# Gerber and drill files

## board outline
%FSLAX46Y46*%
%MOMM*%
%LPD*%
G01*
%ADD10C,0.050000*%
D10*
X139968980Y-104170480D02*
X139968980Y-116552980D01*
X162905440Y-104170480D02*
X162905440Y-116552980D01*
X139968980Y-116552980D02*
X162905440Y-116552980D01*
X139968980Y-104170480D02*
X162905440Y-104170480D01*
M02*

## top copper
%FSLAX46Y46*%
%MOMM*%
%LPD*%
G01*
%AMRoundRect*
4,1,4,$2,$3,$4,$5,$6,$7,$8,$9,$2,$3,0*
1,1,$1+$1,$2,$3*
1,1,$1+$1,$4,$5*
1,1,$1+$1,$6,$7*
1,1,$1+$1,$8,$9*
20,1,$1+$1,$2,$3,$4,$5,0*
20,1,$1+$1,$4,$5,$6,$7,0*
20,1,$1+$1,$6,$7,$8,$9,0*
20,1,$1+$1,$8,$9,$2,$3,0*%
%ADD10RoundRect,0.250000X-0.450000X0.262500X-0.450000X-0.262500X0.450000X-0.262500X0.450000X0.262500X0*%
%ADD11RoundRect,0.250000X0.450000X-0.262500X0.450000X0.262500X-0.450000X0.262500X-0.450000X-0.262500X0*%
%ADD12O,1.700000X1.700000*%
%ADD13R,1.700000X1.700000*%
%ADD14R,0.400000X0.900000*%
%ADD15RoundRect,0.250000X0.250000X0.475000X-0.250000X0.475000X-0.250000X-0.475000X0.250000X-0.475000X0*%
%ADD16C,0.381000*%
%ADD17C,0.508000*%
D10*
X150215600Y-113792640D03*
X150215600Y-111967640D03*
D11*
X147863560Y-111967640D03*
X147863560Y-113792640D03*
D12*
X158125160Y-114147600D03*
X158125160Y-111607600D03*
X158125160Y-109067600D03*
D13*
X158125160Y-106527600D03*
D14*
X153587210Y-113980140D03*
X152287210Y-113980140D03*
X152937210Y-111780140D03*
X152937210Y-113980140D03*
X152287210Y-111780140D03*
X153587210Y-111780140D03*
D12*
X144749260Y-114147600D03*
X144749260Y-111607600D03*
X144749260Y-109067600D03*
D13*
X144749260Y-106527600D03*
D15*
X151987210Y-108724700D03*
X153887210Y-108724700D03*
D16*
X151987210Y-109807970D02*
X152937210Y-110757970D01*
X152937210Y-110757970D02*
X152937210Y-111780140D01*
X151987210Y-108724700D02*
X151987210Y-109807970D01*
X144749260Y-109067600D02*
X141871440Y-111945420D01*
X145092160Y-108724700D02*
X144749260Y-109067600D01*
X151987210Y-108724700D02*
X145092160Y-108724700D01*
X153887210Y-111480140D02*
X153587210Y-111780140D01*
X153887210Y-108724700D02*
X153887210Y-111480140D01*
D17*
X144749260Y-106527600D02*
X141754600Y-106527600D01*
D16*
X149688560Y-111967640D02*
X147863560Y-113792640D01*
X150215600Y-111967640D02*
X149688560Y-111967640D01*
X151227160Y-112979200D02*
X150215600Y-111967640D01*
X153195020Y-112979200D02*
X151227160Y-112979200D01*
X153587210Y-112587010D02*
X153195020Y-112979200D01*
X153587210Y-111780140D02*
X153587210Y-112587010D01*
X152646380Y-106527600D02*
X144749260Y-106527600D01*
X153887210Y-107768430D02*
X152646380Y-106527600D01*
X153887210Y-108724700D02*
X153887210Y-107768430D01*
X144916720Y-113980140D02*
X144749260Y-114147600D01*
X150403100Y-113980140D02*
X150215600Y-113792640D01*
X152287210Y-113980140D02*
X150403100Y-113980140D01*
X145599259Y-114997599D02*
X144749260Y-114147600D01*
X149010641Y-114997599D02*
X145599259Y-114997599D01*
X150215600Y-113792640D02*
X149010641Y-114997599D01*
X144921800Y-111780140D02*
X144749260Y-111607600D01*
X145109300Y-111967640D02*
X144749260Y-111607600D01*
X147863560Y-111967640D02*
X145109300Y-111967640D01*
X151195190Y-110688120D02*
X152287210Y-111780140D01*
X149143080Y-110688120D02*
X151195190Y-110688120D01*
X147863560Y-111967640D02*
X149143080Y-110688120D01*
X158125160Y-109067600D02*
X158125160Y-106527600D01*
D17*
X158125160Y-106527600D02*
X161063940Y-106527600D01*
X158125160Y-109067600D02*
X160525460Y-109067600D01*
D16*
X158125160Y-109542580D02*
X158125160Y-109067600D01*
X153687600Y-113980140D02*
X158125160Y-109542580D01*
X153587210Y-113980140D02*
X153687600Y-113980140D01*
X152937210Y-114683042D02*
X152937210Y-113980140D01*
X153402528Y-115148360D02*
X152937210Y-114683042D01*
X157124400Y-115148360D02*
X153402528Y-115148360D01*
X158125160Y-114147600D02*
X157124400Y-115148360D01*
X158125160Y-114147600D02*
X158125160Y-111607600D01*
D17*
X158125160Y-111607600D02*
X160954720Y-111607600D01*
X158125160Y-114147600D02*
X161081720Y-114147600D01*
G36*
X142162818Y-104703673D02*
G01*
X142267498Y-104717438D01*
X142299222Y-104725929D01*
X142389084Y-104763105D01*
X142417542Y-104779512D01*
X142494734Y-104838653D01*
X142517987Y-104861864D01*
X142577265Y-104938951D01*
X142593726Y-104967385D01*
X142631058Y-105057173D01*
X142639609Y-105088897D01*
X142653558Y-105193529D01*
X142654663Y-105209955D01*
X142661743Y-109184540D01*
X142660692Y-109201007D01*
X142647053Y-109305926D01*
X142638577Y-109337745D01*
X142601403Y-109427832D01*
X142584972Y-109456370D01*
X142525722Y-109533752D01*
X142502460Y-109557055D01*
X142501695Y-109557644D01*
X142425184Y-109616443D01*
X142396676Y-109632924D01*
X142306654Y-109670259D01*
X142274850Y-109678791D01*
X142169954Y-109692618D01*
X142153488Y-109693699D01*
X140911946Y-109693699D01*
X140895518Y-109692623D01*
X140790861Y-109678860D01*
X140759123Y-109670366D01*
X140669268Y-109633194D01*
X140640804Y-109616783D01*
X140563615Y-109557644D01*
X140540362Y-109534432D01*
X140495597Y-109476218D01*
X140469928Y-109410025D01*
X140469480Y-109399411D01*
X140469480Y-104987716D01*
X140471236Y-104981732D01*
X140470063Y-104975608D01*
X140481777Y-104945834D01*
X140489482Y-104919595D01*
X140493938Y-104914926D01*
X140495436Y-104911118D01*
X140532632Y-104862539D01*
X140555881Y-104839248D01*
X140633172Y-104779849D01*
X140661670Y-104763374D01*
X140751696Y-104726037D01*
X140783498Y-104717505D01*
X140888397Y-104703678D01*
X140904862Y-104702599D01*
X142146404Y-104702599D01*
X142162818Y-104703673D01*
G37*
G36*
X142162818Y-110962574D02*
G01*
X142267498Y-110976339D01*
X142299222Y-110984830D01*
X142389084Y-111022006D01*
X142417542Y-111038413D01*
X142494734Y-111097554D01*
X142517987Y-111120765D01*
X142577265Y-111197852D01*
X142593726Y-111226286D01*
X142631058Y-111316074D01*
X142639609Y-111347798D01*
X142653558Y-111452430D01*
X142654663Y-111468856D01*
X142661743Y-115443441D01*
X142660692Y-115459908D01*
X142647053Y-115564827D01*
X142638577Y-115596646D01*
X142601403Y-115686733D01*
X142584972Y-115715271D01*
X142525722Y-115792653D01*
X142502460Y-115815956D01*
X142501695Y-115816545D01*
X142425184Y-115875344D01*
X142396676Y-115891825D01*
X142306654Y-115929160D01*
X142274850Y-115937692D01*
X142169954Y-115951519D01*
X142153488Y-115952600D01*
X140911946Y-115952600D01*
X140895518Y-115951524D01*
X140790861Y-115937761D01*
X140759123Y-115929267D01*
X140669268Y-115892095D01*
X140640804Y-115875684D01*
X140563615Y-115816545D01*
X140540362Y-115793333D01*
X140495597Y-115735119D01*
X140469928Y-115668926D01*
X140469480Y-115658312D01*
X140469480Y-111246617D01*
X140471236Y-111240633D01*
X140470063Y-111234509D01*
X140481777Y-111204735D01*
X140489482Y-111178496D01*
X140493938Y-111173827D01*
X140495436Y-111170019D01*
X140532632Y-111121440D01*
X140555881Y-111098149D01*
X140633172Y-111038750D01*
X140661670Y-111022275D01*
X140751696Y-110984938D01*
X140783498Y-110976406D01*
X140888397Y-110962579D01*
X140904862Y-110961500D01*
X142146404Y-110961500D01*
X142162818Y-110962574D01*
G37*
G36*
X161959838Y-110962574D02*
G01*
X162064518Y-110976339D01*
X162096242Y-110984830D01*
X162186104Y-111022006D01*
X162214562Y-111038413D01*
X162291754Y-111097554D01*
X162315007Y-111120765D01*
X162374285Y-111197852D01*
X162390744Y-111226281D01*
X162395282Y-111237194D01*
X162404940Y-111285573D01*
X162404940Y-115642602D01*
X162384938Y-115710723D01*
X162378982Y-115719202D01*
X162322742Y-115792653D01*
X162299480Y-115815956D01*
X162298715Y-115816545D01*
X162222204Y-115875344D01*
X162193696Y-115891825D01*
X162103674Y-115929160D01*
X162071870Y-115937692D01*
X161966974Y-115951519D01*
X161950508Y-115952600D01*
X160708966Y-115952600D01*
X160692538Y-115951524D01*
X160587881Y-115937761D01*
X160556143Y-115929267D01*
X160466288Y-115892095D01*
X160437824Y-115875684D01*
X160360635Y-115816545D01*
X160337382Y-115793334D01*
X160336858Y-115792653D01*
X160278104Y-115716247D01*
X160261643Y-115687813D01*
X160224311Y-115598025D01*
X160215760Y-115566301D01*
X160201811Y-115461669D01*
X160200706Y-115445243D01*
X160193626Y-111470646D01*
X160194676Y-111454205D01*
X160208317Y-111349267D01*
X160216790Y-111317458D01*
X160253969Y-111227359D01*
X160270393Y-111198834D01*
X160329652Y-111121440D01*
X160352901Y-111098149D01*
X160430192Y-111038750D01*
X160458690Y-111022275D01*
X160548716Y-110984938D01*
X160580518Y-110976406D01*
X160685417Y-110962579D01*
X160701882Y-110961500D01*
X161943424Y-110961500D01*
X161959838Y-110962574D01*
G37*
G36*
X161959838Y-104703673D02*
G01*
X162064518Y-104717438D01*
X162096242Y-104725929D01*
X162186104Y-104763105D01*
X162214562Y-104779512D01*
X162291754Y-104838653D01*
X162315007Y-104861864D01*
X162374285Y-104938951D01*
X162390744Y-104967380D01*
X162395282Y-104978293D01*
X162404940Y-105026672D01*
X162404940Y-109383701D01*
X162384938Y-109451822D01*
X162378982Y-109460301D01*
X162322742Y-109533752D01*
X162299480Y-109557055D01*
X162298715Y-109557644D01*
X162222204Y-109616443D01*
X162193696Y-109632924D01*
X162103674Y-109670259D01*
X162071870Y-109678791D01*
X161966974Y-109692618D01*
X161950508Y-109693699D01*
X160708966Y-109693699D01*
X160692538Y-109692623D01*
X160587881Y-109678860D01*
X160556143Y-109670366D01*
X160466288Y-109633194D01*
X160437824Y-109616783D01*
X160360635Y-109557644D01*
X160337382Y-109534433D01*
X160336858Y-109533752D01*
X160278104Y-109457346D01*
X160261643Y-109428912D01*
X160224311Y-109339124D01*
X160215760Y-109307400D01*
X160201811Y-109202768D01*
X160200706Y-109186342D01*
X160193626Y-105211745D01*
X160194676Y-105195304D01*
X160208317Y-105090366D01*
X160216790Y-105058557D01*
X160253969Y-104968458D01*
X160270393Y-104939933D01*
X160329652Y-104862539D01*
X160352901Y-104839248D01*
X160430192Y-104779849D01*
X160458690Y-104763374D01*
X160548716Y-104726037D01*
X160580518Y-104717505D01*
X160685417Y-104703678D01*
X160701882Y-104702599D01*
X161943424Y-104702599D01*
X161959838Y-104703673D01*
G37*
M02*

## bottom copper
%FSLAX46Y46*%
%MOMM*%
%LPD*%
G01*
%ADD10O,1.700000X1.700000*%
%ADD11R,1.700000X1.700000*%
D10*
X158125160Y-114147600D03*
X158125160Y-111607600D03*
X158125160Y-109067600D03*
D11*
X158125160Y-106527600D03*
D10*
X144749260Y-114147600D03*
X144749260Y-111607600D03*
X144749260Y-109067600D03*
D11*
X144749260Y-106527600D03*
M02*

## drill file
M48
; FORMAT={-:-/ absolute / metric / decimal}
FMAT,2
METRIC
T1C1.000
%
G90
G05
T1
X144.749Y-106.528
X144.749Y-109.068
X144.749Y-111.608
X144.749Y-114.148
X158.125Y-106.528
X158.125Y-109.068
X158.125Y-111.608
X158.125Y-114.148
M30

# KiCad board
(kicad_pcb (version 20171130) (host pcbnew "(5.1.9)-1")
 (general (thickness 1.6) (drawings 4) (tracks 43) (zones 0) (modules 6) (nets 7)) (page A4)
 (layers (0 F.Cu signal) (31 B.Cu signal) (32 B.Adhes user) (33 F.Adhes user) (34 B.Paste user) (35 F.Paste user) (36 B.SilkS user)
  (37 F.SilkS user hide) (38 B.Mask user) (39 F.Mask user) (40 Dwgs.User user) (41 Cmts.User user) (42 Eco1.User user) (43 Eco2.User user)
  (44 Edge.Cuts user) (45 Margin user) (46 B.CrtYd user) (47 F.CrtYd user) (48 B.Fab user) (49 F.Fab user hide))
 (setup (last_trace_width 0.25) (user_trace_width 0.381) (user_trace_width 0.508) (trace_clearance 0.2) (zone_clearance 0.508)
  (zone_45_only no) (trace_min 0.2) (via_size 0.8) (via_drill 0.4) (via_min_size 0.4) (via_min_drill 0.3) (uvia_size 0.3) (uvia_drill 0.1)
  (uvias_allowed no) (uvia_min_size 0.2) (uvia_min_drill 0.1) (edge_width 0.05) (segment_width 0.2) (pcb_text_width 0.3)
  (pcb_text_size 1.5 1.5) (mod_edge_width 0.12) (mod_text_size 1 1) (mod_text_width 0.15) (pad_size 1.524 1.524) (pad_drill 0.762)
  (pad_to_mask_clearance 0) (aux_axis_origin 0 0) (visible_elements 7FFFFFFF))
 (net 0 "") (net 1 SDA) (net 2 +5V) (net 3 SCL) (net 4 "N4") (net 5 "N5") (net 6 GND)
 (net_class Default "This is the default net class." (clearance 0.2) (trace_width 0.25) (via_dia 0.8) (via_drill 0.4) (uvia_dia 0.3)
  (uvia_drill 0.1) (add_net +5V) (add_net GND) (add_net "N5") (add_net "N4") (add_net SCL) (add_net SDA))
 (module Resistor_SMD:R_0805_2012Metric (layer F.Cu) (at 150.2156 112.88014 270)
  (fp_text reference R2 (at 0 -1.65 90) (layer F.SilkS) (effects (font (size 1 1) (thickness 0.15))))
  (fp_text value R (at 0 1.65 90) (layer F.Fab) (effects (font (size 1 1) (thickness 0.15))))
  (pad 2 smd roundrect (at 0.9125 0 270) (size 1.025 1.4) (layers F.Cu F.Paste F.Mask) (roundrect_rratio 0.243902) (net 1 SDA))
  (pad 1 smd roundrect (at -0.9125 0 270) (size 1.025 1.4) (layers F.Cu F.Paste F.Mask) (roundrect_rratio 0.243902) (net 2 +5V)))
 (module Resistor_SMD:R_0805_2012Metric (layer F.Cu) (at 147.86356 112.88014 90)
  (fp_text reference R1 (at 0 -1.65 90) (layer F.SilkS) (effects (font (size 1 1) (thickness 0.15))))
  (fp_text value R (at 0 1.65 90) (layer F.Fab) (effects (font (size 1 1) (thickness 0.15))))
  (pad 2 smd roundrect (at 0.9125 0 90) (size 1.025 1.4) (layers F.Cu F.Paste F.Mask) (roundrect_rratio 0.243902) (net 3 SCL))
  (pad 1 smd roundrect (at -0.9125 0 90) (size 1.025 1.4) (layers F.Cu F.Paste F.Mask) (roundrect_rratio 0.243902) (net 2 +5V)))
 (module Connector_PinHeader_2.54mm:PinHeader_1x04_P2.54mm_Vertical (layer F.Cu) (at 158.12516 106.5276)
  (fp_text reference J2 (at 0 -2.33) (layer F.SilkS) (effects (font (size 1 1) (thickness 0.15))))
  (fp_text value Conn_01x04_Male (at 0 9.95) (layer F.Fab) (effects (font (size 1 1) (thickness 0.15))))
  (pad 4 thru_hole oval (at 0 7.62) (size 1.7 1.7) (drill 1) (layers *.Cu *.Mask) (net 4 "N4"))
  (pad 3 thru_hole oval (at 0 5.08) (size 1.7 1.7) (drill 1) (layers *.Cu *.Mask) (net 4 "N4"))
  (pad 2 thru_hole oval (at 0 2.54) (size 1.7 1.7) (drill 1) (layers *.Cu *.Mask) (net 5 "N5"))
  (pad 1 thru_hole rect (at 0 0) (size 1.7 1.7) (drill 1) (layers *.Cu *.Mask) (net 5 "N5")))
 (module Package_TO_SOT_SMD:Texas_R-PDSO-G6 (layer F.Cu) (at 152.93721 112.88014 270)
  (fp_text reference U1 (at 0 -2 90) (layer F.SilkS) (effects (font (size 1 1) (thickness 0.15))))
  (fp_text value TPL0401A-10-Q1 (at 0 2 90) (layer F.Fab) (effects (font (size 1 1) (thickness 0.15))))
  (pad 6 smd rect (at 1.1 -0.65 270) (size 0.9 0.4) (layers F.Cu F.Paste F.Mask) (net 5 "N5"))
  (pad 4 smd rect (at 1.1 0.65 270) (size 0.9 0.4) (layers F.Cu F.Paste F.Mask) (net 1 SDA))
  (pad 2 smd rect (at -1.1 0 270) (size 0.9 0.4) (layers F.Cu F.Paste F.Mask) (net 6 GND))
  (pad 5 smd rect (at 1.1 0 270) (size 0.9 0.4) (layers F.Cu F.Paste F.Mask) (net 4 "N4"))
  (pad 3 smd rect (at -1.1 0.65 270) (size 0.9 0.4) (layers F.Cu F.Paste F.Mask) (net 3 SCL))
  (pad 1 smd rect (at -1.1 -0.65 270) (size 0.9 0.4) (layers F.Cu F.Paste F.Mask) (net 2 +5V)))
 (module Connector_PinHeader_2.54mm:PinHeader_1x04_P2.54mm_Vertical (layer F.Cu) (at 144.74926 106.5276)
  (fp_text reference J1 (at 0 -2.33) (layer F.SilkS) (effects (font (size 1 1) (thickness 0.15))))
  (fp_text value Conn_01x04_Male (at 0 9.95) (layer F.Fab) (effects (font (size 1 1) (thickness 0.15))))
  (pad 4 thru_hole oval (at 0 7.62) (size 1.7 1.7) (drill 1) (layers *.Cu *.Mask) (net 1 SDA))
  (pad 3 thru_hole oval (at 0 5.08) (size 1.7 1.7) (drill 1) (layers *.Cu *.Mask) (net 3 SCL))
  (pad 2 thru_hole oval (at 0 2.54) (size 1.7 1.7) (drill 1) (layers *.Cu *.Mask) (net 6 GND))
  (pad 1 thru_hole rect (at 0 0) (size 1.7 1.7) (drill 1) (layers *.Cu *.Mask) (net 2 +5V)))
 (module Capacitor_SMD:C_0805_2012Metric (layer F.Cu) (at 152.93721 108.7247 180)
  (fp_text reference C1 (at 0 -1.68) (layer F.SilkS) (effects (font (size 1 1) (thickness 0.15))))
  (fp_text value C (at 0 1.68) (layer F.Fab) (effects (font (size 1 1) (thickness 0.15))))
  (pad 2 smd roundrect (at 0.95 0 180) (size 1 1.45) (layers F.Cu F.Paste F.Mask) (roundrect_rratio 0.25) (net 6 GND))
  (pad 1 smd roundrect (at -0.95 0 180) (size 1 1.45) (layers F.Cu F.Paste F.Mask) (roundrect_rratio 0.25) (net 2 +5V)))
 (gr_line (start 139.96898 104.17048) (end 139.96898 116.55298) (layer Edge.Cuts) (width 0.05))
 (gr_line (start 162.90544 104.17048) (end 162.90544 116.55298) (layer Edge.Cuts) (width 0.05))
 (gr_line (start 139.96898 116.55298) (end 162.90544 116.55298) (layer Edge.Cuts) (width 0.05))
 (gr_line (start 139.96898 104.17048) (end 162.90544 104.17048) (layer Edge.Cuts) (width 0.05))
 (segment (start 151.98721 109.80797) (end 152.93721 110.75797) (width 0.381) (layer F.Cu) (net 6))
 (segment (start 152.93721 110.75797) (end 152.93721 111.78014) (width 0.381) (layer F.Cu) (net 6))
 (segment (start 151.98721 108.7247) (end 151.98721 109.80797) (width 0.381) (layer F.Cu) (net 6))
 (segment (start 144.74926 109.0676) (end 141.87144 111.94542) (width 0.381) (layer F.Cu) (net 6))
 (segment (start 145.09216 108.7247) (end 144.74926 109.0676) (width 0.381) (layer F.Cu) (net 6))
 (segment (start 151.98721 108.7247) (end 145.09216 108.7247) (width 0.381) (layer F.Cu) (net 6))
 (segment (start 153.88721 111.48014) (end 153.58721 111.78014) (width 0.381) (layer F.Cu) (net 2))
 (segment (start 153.88721 108.7247) (end 153.88721 111.48014) (width 0.381) (layer F.Cu) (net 2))
 (segment (start 144.74926 106.5276) (end 141.7546 106.5276) (width 0.508) (layer F.Cu) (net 2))
 (segment (start 149.68856 111.96764) (end 147.86356 113.79264) (width 0.381) (layer F.Cu) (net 2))
 (segment (start 150.2156 111.96764) (end 149.68856 111.96764) (width 0.381) (layer F.Cu) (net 2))
 (segment (start 151.22716 112.9792) (end 150.2156 111.96764) (width 0.381) (layer F.Cu) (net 2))
 (segment (start 153.19502 112.9792) (end 151.22716 112.9792) (width 0.381) (layer F.Cu) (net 2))
 (segment (start 153.58721 112.58701) (end 153.19502 112.9792) (width 0.381) (layer F.Cu) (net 2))
 (segment (start 153.58721 111.78014) (end 153.58721 112.58701) (width 0.381) (layer F.Cu) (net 2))
 (segment (start 152.64638 106.5276) (end 144.74926 106.5276) (width 0.381) (layer F.Cu) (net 2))
 (segment (start 153.88721 107.76843) (end 152.64638 106.5276) (width 0.381) (layer F.Cu) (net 2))
 (segment (start 153.88721 108.7247) (end 153.88721 107.76843) (width 0.381) (layer F.Cu) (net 2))
 (segment (start 144.91672 113.98014) (end 144.74926 114.1476) (width 0.381) (layer F.Cu) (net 1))
 (segment (start 150.4031 113.98014) (end 150.2156 113.79264) (width 0.381) (layer F.Cu) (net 1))
 (segment (start 152.28721 113.98014) (end 150.4031 113.98014) (width 0.381) (layer F.Cu) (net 1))
 (segment (start 145.599259 114.997599) (end 144.74926 114.1476) (width 0.381) (layer F.Cu) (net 1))
 (segment (start 149.010641 114.997599) (end 145.599259 114.997599) (width 0.381) (layer F.Cu) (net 1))
 (segment (start 150.2156 113.79264) (end 149.010641 114.997599) (width 0.381) (layer F.Cu) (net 1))
 (segment (start 144.9218 111.78014) (end 144.74926 111.6076) (width 0.381) (layer F.Cu) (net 3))
 (segment (start 145.1093 111.96764) (end 144.74926 111.6076) (width 0.381) (layer F.Cu) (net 3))
 (segment (start 147.86356 111.96764) (end 145.1093 111.96764) (width 0.381) (layer F.Cu) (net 3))
 (segment (start 151.19519 110.68812) (end 152.28721 111.78014) (width 0.381) (layer F.Cu) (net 3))
 (segment (start 149.14308 110.68812) (end 151.19519 110.68812) (width 0.381) (layer F.Cu) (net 3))
 (segment (start 147.86356 111.96764) (end 149.14308 110.68812) (width 0.381) (layer F.Cu) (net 3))
 (segment (start 158.12516 109.0676) (end 158.12516 106.5276) (width 0.381) (layer F.Cu) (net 5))
 (segment (start 158.12516 106.5276) (end 161.06394 106.5276) (width 0.508) (layer F.Cu) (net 5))
 (segment (start 158.12516 109.0676) (end 160.52546 109.0676) (width 0.508) (layer F.Cu) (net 5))
 (segment (start 158.12516 109.54258) (end 158.12516 109.0676) (width 0.381) (layer F.Cu) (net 5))
 (segment (start 153.6876 113.98014) (end 158.12516 109.54258) (width 0.381) (layer F.Cu) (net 5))
 (segment (start 153.58721 113.98014) (end 153.6876 113.98014) (width 0.381) (layer F.Cu) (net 5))
 (segment (start 152.93721 114.683042) (end 152.93721 113.98014) (width 0.381) (layer F.Cu) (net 4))
 (segment (start 153.402528 115.14836) (end 152.93721 114.683042) (width 0.381) (layer F.Cu) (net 4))
 (segment (start 157.1244 115.14836) (end 153.402528 115.14836) (width 0.381) (layer F.Cu) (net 4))
 (segment (start 158.12516 114.1476) (end 157.1244 115.14836) (width 0.381) (layer F.Cu) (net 4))
 (segment (start 158.12516 114.1476) (end 158.12516 111.6076) (width 0.381) (layer F.Cu) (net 4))
 (segment (start 158.12516 111.6076) (end 160.95472 111.6076) (width 0.508) (layer F.Cu) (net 4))
 (segment (start 158.12516 114.1476) (end 161.08172 114.1476) (width 0.508) (layer F.Cu) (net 4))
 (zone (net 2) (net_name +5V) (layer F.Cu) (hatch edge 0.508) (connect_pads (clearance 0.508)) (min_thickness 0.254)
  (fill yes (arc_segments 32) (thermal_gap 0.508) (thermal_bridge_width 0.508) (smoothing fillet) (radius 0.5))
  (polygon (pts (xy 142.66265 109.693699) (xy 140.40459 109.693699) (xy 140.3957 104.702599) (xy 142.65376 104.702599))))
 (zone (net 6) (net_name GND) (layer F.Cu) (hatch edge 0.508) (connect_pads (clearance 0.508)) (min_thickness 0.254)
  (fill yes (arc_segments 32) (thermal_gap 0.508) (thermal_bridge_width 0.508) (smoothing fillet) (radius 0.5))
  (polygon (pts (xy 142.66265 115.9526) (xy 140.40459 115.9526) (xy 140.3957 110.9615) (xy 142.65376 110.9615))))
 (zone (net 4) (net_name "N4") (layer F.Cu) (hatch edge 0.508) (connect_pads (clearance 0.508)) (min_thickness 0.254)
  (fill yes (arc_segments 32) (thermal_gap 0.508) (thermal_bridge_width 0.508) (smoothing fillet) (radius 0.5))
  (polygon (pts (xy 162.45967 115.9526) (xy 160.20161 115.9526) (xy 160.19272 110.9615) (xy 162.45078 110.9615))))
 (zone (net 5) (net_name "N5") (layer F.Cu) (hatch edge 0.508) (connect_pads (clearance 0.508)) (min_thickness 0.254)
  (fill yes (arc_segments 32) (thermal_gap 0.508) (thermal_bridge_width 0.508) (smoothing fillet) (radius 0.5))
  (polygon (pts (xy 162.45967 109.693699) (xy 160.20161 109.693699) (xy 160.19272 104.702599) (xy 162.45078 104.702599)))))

